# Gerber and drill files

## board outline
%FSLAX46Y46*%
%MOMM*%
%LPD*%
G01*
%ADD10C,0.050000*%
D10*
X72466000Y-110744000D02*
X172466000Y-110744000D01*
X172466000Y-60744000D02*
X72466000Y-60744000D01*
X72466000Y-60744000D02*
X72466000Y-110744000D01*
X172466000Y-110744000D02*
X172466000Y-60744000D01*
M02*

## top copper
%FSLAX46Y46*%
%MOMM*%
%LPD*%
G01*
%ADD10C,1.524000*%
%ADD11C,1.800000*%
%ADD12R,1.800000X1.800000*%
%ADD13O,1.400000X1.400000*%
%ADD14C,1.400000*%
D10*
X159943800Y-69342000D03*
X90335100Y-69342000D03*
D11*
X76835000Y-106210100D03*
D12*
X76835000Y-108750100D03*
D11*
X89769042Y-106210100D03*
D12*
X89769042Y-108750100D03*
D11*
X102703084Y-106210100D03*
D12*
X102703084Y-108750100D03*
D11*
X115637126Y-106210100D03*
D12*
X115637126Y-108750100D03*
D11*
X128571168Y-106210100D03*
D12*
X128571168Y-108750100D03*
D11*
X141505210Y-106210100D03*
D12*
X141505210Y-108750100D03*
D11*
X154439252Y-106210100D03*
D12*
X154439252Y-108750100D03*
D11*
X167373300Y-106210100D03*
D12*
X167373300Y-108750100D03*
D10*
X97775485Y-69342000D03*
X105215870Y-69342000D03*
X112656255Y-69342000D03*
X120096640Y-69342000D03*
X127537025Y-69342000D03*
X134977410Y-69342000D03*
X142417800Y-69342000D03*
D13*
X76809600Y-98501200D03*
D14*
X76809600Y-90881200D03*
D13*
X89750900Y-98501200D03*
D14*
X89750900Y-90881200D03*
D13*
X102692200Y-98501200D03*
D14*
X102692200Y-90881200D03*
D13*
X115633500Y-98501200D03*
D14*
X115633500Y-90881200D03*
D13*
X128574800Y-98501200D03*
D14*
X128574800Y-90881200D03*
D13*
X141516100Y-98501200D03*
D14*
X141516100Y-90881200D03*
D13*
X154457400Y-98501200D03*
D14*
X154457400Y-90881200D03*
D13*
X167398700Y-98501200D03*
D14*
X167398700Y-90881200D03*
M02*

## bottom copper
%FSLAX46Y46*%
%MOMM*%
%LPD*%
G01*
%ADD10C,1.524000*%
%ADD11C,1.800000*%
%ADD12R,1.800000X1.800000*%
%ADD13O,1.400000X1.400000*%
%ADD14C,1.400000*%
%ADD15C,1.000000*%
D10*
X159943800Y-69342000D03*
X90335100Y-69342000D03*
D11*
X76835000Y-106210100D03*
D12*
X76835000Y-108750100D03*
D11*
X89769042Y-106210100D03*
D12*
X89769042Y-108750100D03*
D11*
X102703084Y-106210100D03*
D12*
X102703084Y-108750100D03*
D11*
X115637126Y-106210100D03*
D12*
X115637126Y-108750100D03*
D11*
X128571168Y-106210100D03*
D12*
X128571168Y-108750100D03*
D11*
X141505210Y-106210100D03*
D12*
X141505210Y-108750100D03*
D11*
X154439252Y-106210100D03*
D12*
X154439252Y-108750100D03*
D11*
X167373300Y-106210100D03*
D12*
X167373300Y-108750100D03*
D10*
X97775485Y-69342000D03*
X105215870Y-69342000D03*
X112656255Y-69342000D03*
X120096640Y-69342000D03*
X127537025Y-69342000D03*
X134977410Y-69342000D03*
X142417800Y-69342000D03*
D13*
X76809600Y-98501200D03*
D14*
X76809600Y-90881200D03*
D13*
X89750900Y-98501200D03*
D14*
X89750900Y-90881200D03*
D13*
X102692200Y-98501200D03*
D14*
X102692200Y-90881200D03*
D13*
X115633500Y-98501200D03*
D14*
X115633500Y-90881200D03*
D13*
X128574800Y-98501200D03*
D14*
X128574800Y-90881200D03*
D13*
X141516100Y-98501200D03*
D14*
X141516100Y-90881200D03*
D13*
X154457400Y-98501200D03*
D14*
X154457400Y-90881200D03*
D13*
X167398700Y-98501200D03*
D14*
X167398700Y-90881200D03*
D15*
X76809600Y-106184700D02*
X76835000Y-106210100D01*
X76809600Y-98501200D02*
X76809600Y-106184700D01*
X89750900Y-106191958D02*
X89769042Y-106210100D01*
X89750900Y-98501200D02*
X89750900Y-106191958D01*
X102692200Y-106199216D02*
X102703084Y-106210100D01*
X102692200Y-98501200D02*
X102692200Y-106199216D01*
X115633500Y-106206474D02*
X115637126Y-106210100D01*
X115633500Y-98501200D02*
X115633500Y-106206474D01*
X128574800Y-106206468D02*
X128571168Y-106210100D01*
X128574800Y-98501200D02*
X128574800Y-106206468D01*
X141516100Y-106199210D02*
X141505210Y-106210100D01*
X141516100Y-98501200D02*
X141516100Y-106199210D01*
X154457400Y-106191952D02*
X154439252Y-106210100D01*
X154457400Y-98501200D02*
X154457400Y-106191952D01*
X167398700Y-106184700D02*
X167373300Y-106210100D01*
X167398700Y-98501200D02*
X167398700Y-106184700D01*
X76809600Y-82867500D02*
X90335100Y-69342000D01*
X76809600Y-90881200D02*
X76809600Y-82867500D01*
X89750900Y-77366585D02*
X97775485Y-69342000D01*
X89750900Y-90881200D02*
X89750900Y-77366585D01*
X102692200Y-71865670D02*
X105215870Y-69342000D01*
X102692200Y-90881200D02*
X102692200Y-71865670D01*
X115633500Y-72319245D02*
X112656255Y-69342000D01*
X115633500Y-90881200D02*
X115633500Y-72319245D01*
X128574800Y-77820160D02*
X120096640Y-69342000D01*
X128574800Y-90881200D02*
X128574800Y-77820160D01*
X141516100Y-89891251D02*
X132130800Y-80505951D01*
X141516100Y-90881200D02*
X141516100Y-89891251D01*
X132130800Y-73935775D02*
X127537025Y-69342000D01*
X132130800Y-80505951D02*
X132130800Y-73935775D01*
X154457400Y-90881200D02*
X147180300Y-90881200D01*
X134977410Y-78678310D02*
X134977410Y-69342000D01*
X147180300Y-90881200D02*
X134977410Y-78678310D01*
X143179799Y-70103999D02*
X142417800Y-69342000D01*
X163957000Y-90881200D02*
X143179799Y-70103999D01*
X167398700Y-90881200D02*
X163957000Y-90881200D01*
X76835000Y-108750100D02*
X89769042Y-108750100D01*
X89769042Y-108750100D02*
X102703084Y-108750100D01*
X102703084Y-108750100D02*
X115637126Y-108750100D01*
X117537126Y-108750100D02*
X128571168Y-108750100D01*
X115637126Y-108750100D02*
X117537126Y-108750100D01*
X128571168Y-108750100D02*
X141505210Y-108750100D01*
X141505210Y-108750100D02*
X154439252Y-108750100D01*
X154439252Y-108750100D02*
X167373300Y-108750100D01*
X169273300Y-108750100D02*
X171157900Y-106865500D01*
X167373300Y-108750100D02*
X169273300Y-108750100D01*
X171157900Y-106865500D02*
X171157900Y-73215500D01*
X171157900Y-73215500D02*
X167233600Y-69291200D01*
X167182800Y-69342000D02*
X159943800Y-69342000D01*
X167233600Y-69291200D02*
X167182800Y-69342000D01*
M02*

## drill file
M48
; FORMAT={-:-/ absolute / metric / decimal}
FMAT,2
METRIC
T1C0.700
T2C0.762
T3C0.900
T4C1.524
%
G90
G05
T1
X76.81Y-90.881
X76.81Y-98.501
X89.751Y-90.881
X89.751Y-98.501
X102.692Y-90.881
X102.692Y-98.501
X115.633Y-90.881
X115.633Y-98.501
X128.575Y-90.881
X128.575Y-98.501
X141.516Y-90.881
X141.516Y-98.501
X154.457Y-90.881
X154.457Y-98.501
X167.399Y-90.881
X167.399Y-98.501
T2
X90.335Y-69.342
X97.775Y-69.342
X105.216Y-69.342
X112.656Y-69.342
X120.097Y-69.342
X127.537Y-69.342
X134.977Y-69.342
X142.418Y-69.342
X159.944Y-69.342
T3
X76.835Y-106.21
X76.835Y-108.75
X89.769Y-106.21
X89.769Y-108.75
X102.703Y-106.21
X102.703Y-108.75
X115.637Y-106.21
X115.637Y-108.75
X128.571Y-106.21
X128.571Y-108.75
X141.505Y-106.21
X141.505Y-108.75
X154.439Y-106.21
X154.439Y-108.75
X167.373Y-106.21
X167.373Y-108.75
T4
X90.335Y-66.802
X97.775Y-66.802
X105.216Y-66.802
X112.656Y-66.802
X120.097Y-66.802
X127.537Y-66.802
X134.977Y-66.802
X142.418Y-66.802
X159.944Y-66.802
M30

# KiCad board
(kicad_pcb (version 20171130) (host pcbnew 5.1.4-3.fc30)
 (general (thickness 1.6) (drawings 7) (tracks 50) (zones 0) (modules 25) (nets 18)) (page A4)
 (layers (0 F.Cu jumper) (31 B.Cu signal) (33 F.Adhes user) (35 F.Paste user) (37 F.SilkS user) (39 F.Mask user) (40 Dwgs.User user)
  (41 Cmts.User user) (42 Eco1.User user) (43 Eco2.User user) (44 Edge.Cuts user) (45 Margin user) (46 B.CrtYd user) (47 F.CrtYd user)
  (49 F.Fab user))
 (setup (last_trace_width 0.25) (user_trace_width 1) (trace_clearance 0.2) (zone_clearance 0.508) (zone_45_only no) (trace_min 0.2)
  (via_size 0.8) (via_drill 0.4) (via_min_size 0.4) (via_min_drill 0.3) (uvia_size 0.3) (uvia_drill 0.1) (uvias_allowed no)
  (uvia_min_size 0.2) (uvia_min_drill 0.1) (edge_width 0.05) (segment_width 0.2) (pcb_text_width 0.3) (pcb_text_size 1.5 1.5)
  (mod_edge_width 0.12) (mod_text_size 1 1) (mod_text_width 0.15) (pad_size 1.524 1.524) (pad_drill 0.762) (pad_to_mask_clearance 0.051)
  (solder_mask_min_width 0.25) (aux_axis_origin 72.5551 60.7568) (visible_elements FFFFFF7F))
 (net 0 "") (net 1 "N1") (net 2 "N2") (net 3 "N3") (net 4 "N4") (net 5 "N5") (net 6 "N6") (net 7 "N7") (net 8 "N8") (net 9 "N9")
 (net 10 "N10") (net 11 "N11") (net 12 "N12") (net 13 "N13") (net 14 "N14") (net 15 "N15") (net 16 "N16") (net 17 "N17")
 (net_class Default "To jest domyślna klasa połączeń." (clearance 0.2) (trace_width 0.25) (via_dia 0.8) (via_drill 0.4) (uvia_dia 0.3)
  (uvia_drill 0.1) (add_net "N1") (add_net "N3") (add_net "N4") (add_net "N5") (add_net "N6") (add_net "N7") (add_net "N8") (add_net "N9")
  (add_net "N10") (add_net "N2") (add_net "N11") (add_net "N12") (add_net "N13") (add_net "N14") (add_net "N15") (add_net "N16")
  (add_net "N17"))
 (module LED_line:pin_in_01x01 (layer F.Cu) (at 159.9438 69.342 180)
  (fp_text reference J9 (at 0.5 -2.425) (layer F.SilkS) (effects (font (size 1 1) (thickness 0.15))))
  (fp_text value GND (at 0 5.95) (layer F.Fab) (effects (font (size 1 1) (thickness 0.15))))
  (pad "" np_thru_hole circle (at 0 2.54 180) (size 1.524 1.524) (drill 1.524) (layers *.Cu *.Mask))
  (pad 1 thru_hole circle (at 0 0 180) (size 1.524 1.524) (drill 0.762) (layers *.Mask B.Cu) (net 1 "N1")))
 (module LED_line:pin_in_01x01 (layer F.Cu) (at 90.3351 69.342 180)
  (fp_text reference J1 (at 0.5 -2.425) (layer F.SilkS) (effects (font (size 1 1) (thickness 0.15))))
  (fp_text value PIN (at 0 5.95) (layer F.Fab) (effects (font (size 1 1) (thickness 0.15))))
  (pad "" np_thru_hole circle (at 0 2.54 180) (size 1.524 1.524) (drill 1.524) (layers *.Cu *.Mask))
  (pad 1 thru_hole circle (at 0 0 180) (size 1.524 1.524) (drill 0.762) (layers *.Mask B.Cu) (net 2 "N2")))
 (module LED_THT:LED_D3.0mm (layer F.Cu) (at 76.835 108.7501 90)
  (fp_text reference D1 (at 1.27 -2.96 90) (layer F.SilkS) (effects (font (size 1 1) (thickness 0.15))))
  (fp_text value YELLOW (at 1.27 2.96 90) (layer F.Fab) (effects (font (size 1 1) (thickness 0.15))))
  (pad 2 thru_hole circle (at 2.54 0 90) (size 1.8 1.8) (drill 0.9) (layers *.Cu *.Mask) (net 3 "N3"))
  (pad 1 thru_hole rect (at 0 0 90) (size 1.8 1.8) (drill 0.9) (layers *.Cu *.Mask) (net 1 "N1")))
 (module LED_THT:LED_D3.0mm (layer F.Cu) (at 89.769042 108.7501 90)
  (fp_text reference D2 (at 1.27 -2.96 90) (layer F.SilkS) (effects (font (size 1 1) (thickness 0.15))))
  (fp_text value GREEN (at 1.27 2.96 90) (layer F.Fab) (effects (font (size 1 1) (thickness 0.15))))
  (pad 2 thru_hole circle (at 2.54 0 90) (size 1.8 1.8) (drill 0.9) (layers *.Cu *.Mask) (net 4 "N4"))
  (pad 1 thru_hole rect (at 0 0 90) (size 1.8 1.8) (drill 0.9) (layers *.Cu *.Mask) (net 1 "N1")))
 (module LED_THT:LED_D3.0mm (layer F.Cu) (at 102.703084 108.7501 90)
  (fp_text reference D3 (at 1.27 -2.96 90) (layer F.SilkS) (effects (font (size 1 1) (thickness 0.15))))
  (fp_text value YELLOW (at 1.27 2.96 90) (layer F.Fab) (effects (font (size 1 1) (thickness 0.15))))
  (pad 2 thru_hole circle (at 2.54 0 90) (size 1.8 1.8) (drill 0.9) (layers *.Cu *.Mask) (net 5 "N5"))
  (pad 1 thru_hole rect (at 0 0 90) (size 1.8 1.8) (drill 0.9) (layers *.Cu *.Mask) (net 1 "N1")))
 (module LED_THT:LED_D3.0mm (layer F.Cu) (at 115.637126 108.7501 90)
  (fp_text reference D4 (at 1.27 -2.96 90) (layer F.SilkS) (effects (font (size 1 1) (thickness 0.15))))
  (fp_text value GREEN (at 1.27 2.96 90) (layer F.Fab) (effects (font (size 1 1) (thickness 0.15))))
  (pad 2 thru_hole circle (at 2.54 0 90) (size 1.8 1.8) (drill 0.9) (layers *.Cu *.Mask) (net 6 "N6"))
  (pad 1 thru_hole rect (at 0 0 90) (size 1.8 1.8) (drill 0.9) (layers *.Cu *.Mask) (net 1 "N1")))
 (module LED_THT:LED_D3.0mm (layer F.Cu) (at 128.571168 108.7501 90)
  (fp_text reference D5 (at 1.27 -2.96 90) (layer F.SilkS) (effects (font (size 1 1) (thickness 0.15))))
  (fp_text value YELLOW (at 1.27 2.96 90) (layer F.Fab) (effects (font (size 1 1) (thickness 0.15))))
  (pad 2 thru_hole circle (at 2.54 0 90) (size 1.8 1.8) (drill 0.9) (layers *.Cu *.Mask) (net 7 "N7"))
  (pad 1 thru_hole rect (at 0 0 90) (size 1.8 1.8) (drill 0.9) (layers *.Cu *.Mask) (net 1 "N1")))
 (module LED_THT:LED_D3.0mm (layer F.Cu) (at 141.50521 108.7501 90)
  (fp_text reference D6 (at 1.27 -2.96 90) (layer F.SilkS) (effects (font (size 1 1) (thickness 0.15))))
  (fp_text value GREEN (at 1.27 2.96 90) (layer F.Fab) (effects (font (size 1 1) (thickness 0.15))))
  (pad 2 thru_hole circle (at 2.54 0 90) (size 1.8 1.8) (drill 0.9) (layers *.Cu *.Mask) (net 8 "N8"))
  (pad 1 thru_hole rect (at 0 0 90) (size 1.8 1.8) (drill 0.9) (layers *.Cu *.Mask) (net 1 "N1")))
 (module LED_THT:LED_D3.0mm (layer F.Cu) (at 154.439252 108.7501 90)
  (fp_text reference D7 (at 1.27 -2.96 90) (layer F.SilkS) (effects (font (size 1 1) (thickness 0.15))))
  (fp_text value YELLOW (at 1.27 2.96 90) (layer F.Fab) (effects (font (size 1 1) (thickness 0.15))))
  (pad 2 thru_hole circle (at 2.54 0 90) (size 1.8 1.8) (drill 0.9) (layers *.Cu *.Mask) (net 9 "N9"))
  (pad 1 thru_hole rect (at 0 0 90) (size 1.8 1.8) (drill 0.9) (layers *.Cu *.Mask) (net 1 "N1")))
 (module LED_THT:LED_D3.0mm (layer F.Cu) (at 167.3733 108.7501 90)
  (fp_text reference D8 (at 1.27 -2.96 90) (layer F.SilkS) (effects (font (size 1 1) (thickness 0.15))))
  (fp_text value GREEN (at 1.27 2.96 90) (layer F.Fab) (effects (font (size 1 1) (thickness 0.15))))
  (pad 2 thru_hole circle (at 2.54 0 90) (size 1.8 1.8) (drill 0.9) (layers *.Cu *.Mask) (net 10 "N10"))
  (pad 1 thru_hole rect (at 0 0 90) (size 1.8 1.8) (drill 0.9) (layers *.Cu *.Mask) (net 1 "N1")))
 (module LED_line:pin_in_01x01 (layer F.Cu) (at 97.775485 69.342 180)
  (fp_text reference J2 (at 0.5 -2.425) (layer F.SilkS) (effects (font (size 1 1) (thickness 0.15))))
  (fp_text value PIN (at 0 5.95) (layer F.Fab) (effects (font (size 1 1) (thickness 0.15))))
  (pad "" np_thru_hole circle (at 0 2.54 180) (size 1.524 1.524) (drill 1.524) (layers *.Cu *.Mask))
  (pad 1 thru_hole circle (at 0 0 180) (size 1.524 1.524) (drill 0.762) (layers *.Mask B.Cu) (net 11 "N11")))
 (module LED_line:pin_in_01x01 (layer F.Cu) (at 105.21587 69.342 180)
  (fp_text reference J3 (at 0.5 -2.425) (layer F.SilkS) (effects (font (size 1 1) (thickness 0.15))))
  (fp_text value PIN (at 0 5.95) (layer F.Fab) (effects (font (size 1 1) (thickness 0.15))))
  (pad "" np_thru_hole circle (at 0 2.54 180) (size 1.524 1.524) (drill 1.524) (layers *.Cu *.Mask))
  (pad 1 thru_hole circle (at 0 0 180) (size 1.524 1.524) (drill 0.762) (layers *.Mask B.Cu) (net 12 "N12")))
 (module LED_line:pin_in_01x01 (layer F.Cu) (at 112.656255 69.342 180)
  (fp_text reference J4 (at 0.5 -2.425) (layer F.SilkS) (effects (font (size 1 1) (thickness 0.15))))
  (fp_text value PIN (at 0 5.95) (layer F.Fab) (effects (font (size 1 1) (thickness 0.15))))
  (pad "" np_thru_hole circle (at 0 2.54 180) (size 1.524 1.524) (drill 1.524) (layers *.Cu *.Mask))
  (pad 1 thru_hole circle (at 0 0 180) (size 1.524 1.524) (drill 0.762) (layers *.Mask B.Cu) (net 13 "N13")))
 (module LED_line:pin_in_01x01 (layer F.Cu) (at 120.09664 69.342 180)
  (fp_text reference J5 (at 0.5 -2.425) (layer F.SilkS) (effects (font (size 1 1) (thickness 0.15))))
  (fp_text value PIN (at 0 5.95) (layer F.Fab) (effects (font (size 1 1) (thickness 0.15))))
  (pad "" np_thru_hole circle (at 0 2.54 180) (size 1.524 1.524) (drill 1.524) (layers *.Cu *.Mask))
  (pad 1 thru_hole circle (at 0 0 180) (size 1.524 1.524) (drill 0.762) (layers *.Mask B.Cu) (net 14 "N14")))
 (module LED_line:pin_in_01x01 (layer F.Cu) (at 127.537025 69.342 180)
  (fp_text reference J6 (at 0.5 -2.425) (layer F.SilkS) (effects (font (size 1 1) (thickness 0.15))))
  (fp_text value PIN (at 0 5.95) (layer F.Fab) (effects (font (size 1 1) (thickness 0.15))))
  (pad "" np_thru_hole circle (at 0 2.54 180) (size 1.524 1.524) (drill 1.524) (layers *.Cu *.Mask))
  (pad 1 thru_hole circle (at 0 0 180) (size 1.524 1.524) (drill 0.762) (layers *.Mask B.Cu) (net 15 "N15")))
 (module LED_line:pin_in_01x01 (layer F.Cu) (at 134.97741 69.342 180)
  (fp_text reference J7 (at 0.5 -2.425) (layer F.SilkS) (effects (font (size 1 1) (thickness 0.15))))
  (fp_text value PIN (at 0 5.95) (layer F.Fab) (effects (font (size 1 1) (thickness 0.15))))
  (pad "" np_thru_hole circle (at 0 2.54 180) (size 1.524 1.524) (drill 1.524) (layers *.Cu *.Mask))
  (pad 1 thru_hole circle (at 0 0 180) (size 1.524 1.524) (drill 0.762) (layers *.Mask B.Cu) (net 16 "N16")))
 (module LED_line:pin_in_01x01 (layer F.Cu) (at 142.4178 69.342 180)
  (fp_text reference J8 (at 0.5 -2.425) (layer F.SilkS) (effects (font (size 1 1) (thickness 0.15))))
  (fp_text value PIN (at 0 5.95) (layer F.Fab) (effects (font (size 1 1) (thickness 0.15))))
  (pad "" np_thru_hole circle (at 0 2.54 180) (size 1.524 1.524) (drill 1.524) (layers *.Cu *.Mask))
  (pad 1 thru_hole circle (at 0 0 180) (size 1.524 1.524) (drill 0.762) (layers *.Mask B.Cu) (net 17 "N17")))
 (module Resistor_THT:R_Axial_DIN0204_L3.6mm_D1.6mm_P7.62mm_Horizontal (layer F.Cu) (at 76.8096 90.8812 270)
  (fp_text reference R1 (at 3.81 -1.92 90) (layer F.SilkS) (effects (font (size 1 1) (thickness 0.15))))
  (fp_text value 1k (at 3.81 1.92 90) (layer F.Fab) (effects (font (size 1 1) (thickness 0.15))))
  (pad 2 thru_hole oval (at 7.62 0 270) (size 1.4 1.4) (drill 0.7) (layers *.Cu *.Mask) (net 3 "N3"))
  (pad 1 thru_hole circle (at 0 0 270) (size 1.4 1.4) (drill 0.7) (layers *.Cu *.Mask) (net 2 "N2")))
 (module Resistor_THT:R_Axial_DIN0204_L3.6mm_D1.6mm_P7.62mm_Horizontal (layer F.Cu) (at 89.7509 90.8812 270)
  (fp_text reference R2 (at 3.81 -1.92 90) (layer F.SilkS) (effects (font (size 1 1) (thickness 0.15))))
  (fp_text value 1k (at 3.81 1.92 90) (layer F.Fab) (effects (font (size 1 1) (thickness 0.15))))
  (pad 2 thru_hole oval (at 7.62 0 270) (size 1.4 1.4) (drill 0.7) (layers *.Cu *.Mask) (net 4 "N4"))
  (pad 1 thru_hole circle (at 0 0 270) (size 1.4 1.4) (drill 0.7) (layers *.Cu *.Mask) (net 11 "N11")))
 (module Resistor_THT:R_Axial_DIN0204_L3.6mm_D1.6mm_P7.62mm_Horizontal (layer F.Cu) (at 102.6922 90.8812 270)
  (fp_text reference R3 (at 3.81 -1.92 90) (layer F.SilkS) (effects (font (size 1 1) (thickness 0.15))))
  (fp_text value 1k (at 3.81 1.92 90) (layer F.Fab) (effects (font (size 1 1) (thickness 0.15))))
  (pad 2 thru_hole oval (at 7.62 0 270) (size 1.4 1.4) (drill 0.7) (layers *.Cu *.Mask) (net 5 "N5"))
  (pad 1 thru_hole circle (at 0 0 270) (size 1.4 1.4) (drill 0.7) (layers *.Cu *.Mask) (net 12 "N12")))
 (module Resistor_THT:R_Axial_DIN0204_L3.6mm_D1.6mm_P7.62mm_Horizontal (layer F.Cu) (at 115.6335 90.8812 270)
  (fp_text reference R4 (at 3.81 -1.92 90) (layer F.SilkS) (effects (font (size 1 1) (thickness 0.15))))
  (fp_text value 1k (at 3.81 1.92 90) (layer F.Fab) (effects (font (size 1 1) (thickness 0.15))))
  (pad 2 thru_hole oval (at 7.62 0 270) (size 1.4 1.4) (drill 0.7) (layers *.Cu *.Mask) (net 6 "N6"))
  (pad 1 thru_hole circle (at 0 0 270) (size 1.4 1.4) (drill 0.7) (layers *.Cu *.Mask) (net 13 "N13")))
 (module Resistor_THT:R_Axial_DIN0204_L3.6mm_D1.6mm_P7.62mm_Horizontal (layer F.Cu) (at 128.5748 90.8812 270)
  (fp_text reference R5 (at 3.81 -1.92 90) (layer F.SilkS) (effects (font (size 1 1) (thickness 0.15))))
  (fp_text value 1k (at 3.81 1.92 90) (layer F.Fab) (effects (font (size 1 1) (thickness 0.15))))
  (pad 2 thru_hole oval (at 7.62 0 270) (size 1.4 1.4) (drill 0.7) (layers *.Cu *.Mask) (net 7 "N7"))
  (pad 1 thru_hole circle (at 0 0 270) (size 1.4 1.4) (drill 0.7) (layers *.Cu *.Mask) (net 14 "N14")))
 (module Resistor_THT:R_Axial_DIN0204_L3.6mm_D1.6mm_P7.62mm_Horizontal (layer F.Cu) (at 141.5161 90.8812 270)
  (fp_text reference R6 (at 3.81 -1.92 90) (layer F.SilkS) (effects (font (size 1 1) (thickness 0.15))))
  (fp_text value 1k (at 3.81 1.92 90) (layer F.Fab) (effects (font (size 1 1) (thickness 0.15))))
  (pad 2 thru_hole oval (at 7.62 0 270) (size 1.4 1.4) (drill 0.7) (layers *.Cu *.Mask) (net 8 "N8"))
  (pad 1 thru_hole circle (at 0 0 270) (size 1.4 1.4) (drill 0.7) (layers *.Cu *.Mask) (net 15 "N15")))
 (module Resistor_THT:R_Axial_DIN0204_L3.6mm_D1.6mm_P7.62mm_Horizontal (layer F.Cu) (at 154.4574 90.8812 270)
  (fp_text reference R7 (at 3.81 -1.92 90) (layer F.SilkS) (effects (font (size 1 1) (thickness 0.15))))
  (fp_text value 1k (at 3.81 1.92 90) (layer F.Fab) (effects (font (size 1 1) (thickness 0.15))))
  (pad 2 thru_hole oval (at 7.62 0 270) (size 1.4 1.4) (drill 0.7) (layers *.Cu *.Mask) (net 9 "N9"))
  (pad 1 thru_hole circle (at 0 0 270) (size 1.4 1.4) (drill 0.7) (layers *.Cu *.Mask) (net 16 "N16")))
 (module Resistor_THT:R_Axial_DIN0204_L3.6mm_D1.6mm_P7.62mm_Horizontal (layer F.Cu) (at 167.3987 90.8812 270)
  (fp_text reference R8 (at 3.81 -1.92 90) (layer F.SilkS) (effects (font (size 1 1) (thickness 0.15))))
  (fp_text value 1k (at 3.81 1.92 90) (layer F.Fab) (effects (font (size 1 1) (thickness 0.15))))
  (pad 2 thru_hole oval (at 7.62 0 270) (size 1.4 1.4) (drill 0.7) (layers *.Cu *.Mask) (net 10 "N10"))
  (pad 1 thru_hole circle (at 0 0 270) (size 1.4 1.4) (drill 0.7) (layers *.Cu *.Mask) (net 17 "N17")))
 (gr_line (start 72.466 110.744) (end 172.466 110.744) (layer Edge.Cuts) (width 0.05))
 (gr_line (start 172.466 60.744) (end 72.466 60.744) (layer Edge.Cuts) (width 0.05))
 (gr_line (start 72.466 60.744) (end 72.466 110.744) (layer Edge.Cuts) (width 0.05))
 (gr_line (start 172.466 110.744) (end 172.466 60.744) (layer Edge.Cuts) (width 0.05))
 (segment (start 76.8096 106.1847) (end 76.835 106.2101) (width 1) (layer B.Cu) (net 3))
 (segment (start 76.8096 98.5012) (end 76.8096 106.1847) (width 1) (layer B.Cu) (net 3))
 (segment (start 89.7509 106.191958) (end 89.769042 106.2101) (width 1) (layer B.Cu) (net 4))
 (segment (start 89.7509 98.5012) (end 89.7509 106.191958) (width 1) (layer B.Cu) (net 4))
 (segment (start 102.6922 106.199216) (end 102.703084 106.2101) (width 1) (layer B.Cu) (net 5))
 (segment (start 102.6922 98.5012) (end 102.6922 106.199216) (width 1) (layer B.Cu) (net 5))
 (segment (start 115.6335 106.206474) (end 115.637126 106.2101) (width 1) (layer B.Cu) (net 6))
 (segment (start 115.6335 98.5012) (end 115.6335 106.206474) (width 1) (layer B.Cu) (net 6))
 (segment (start 128.5748 106.206468) (end 128.571168 106.2101) (width 1) (layer B.Cu) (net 7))
 (segment (start 128.5748 98.5012) (end 128.5748 106.206468) (width 1) (layer B.Cu) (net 7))
 (segment (start 141.5161 106.19921) (end 141.50521 106.2101) (width 1) (layer B.Cu) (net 8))
 (segment (start 141.5161 98.5012) (end 141.5161 106.19921) (width 1) (layer B.Cu) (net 8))
 (segment (start 154.4574 106.191952) (end 154.439252 106.2101) (width 1) (layer B.Cu) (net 9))
 (segment (start 154.4574 98.5012) (end 154.4574 106.191952) (width 1) (layer B.Cu) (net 9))
 (segment (start 167.3987 106.1847) (end 167.3733 106.2101) (width 1) (layer B.Cu) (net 10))
 (segment (start 167.3987 98.5012) (end 167.3987 106.1847) (width 1) (layer B.Cu) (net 10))
 (segment (start 76.8096 82.8675) (end 90.3351 69.342) (width 1) (layer B.Cu) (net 2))
 (segment (start 76.8096 90.8812) (end 76.8096 82.8675) (width 1) (layer B.Cu) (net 2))
 (segment (start 89.7509 77.366585) (end 97.775485 69.342) (width 1) (layer B.Cu) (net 11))
 (segment (start 89.7509 90.8812) (end 89.7509 77.366585) (width 1) (layer B.Cu) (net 11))
 (segment (start 102.6922 71.86567) (end 105.21587 69.342) (width 1) (layer B.Cu) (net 12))
 (segment (start 102.6922 90.8812) (end 102.6922 71.86567) (width 1) (layer B.Cu) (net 12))
 (segment (start 115.6335 72.319245) (end 112.656255 69.342) (width 1) (layer B.Cu) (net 13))
 (segment (start 115.6335 90.8812) (end 115.6335 72.319245) (width 1) (layer B.Cu) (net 13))
 (segment (start 128.5748 77.82016) (end 120.09664 69.342) (width 1) (layer B.Cu) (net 14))
 (segment (start 128.5748 90.8812) (end 128.5748 77.82016) (width 1) (layer B.Cu) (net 14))
 (segment (start 141.5161 89.891251) (end 132.1308 80.505951) (width 1) (layer B.Cu) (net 15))
 (segment (start 141.5161 90.8812) (end 141.5161 89.891251) (width 1) (layer B.Cu) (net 15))
 (segment (start 132.1308 73.935775) (end 127.537025 69.342) (width 1) (layer B.Cu) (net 15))
 (segment (start 132.1308 80.505951) (end 132.1308 73.935775) (width 1) (layer B.Cu) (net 15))
 (segment (start 154.4574 90.8812) (end 147.1803 90.8812) (width 1) (layer B.Cu) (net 16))
 (segment (start 134.97741 78.67831) (end 134.97741 69.342) (width 1) (layer B.Cu) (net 16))
 (segment (start 147.1803 90.8812) (end 134.97741 78.67831) (width 1) (layer B.Cu) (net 16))
 (segment (start 143.179799 70.103999) (end 142.4178 69.342) (width 1) (layer B.Cu) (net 17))
 (segment (start 163.957 90.8812) (end 143.179799 70.103999) (width 1) (layer B.Cu) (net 17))
 (segment (start 167.3987 90.8812) (end 163.957 90.8812) (width 1) (layer B.Cu) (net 17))
 (segment (start 76.835 108.7501) (end 89.769042 108.7501) (width 1) (layer B.Cu) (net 1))
 (segment (start 89.769042 108.7501) (end 102.703084 108.7501) (width 1) (layer B.Cu) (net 1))
 (segment (start 102.703084 108.7501) (end 115.637126 108.7501) (width 1) (layer B.Cu) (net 1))
 (segment (start 117.537126 108.7501) (end 128.571168 108.7501) (width 1) (layer B.Cu) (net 1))
 (segment (start 115.637126 108.7501) (end 117.537126 108.7501) (width 1) (layer B.Cu) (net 1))
 (segment (start 128.571168 108.7501) (end 141.50521 108.7501) (width 1) (layer B.Cu) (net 1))
 (segment (start 141.50521 108.7501) (end 154.439252 108.7501) (width 1) (layer B.Cu) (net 1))
 (segment (start 154.439252 108.7501) (end 167.3733 108.7501) (width 1) (layer B.Cu) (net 1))
 (segment (start 169.2733 108.7501) (end 171.1579 106.8655) (width 1) (layer B.Cu) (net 1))
 (segment (start 167.3733 108.7501) (end 169.2733 108.7501) (width 1) (layer B.Cu) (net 1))
 (segment (start 171.1579 106.8655) (end 171.1579 73.2155) (width 1) (layer B.Cu) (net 1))
 (segment (start 171.1579 73.2155) (end 167.2336 69.2912) (width 1) (layer B.Cu) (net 1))
 (segment (start 167.1828 69.342) (end 159.9438 69.342) (width 1) (layer B.Cu) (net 1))
 (segment (start 167.2336 69.2912) (end 167.1828 69.342) (width 1) (layer B.Cu) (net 1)))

